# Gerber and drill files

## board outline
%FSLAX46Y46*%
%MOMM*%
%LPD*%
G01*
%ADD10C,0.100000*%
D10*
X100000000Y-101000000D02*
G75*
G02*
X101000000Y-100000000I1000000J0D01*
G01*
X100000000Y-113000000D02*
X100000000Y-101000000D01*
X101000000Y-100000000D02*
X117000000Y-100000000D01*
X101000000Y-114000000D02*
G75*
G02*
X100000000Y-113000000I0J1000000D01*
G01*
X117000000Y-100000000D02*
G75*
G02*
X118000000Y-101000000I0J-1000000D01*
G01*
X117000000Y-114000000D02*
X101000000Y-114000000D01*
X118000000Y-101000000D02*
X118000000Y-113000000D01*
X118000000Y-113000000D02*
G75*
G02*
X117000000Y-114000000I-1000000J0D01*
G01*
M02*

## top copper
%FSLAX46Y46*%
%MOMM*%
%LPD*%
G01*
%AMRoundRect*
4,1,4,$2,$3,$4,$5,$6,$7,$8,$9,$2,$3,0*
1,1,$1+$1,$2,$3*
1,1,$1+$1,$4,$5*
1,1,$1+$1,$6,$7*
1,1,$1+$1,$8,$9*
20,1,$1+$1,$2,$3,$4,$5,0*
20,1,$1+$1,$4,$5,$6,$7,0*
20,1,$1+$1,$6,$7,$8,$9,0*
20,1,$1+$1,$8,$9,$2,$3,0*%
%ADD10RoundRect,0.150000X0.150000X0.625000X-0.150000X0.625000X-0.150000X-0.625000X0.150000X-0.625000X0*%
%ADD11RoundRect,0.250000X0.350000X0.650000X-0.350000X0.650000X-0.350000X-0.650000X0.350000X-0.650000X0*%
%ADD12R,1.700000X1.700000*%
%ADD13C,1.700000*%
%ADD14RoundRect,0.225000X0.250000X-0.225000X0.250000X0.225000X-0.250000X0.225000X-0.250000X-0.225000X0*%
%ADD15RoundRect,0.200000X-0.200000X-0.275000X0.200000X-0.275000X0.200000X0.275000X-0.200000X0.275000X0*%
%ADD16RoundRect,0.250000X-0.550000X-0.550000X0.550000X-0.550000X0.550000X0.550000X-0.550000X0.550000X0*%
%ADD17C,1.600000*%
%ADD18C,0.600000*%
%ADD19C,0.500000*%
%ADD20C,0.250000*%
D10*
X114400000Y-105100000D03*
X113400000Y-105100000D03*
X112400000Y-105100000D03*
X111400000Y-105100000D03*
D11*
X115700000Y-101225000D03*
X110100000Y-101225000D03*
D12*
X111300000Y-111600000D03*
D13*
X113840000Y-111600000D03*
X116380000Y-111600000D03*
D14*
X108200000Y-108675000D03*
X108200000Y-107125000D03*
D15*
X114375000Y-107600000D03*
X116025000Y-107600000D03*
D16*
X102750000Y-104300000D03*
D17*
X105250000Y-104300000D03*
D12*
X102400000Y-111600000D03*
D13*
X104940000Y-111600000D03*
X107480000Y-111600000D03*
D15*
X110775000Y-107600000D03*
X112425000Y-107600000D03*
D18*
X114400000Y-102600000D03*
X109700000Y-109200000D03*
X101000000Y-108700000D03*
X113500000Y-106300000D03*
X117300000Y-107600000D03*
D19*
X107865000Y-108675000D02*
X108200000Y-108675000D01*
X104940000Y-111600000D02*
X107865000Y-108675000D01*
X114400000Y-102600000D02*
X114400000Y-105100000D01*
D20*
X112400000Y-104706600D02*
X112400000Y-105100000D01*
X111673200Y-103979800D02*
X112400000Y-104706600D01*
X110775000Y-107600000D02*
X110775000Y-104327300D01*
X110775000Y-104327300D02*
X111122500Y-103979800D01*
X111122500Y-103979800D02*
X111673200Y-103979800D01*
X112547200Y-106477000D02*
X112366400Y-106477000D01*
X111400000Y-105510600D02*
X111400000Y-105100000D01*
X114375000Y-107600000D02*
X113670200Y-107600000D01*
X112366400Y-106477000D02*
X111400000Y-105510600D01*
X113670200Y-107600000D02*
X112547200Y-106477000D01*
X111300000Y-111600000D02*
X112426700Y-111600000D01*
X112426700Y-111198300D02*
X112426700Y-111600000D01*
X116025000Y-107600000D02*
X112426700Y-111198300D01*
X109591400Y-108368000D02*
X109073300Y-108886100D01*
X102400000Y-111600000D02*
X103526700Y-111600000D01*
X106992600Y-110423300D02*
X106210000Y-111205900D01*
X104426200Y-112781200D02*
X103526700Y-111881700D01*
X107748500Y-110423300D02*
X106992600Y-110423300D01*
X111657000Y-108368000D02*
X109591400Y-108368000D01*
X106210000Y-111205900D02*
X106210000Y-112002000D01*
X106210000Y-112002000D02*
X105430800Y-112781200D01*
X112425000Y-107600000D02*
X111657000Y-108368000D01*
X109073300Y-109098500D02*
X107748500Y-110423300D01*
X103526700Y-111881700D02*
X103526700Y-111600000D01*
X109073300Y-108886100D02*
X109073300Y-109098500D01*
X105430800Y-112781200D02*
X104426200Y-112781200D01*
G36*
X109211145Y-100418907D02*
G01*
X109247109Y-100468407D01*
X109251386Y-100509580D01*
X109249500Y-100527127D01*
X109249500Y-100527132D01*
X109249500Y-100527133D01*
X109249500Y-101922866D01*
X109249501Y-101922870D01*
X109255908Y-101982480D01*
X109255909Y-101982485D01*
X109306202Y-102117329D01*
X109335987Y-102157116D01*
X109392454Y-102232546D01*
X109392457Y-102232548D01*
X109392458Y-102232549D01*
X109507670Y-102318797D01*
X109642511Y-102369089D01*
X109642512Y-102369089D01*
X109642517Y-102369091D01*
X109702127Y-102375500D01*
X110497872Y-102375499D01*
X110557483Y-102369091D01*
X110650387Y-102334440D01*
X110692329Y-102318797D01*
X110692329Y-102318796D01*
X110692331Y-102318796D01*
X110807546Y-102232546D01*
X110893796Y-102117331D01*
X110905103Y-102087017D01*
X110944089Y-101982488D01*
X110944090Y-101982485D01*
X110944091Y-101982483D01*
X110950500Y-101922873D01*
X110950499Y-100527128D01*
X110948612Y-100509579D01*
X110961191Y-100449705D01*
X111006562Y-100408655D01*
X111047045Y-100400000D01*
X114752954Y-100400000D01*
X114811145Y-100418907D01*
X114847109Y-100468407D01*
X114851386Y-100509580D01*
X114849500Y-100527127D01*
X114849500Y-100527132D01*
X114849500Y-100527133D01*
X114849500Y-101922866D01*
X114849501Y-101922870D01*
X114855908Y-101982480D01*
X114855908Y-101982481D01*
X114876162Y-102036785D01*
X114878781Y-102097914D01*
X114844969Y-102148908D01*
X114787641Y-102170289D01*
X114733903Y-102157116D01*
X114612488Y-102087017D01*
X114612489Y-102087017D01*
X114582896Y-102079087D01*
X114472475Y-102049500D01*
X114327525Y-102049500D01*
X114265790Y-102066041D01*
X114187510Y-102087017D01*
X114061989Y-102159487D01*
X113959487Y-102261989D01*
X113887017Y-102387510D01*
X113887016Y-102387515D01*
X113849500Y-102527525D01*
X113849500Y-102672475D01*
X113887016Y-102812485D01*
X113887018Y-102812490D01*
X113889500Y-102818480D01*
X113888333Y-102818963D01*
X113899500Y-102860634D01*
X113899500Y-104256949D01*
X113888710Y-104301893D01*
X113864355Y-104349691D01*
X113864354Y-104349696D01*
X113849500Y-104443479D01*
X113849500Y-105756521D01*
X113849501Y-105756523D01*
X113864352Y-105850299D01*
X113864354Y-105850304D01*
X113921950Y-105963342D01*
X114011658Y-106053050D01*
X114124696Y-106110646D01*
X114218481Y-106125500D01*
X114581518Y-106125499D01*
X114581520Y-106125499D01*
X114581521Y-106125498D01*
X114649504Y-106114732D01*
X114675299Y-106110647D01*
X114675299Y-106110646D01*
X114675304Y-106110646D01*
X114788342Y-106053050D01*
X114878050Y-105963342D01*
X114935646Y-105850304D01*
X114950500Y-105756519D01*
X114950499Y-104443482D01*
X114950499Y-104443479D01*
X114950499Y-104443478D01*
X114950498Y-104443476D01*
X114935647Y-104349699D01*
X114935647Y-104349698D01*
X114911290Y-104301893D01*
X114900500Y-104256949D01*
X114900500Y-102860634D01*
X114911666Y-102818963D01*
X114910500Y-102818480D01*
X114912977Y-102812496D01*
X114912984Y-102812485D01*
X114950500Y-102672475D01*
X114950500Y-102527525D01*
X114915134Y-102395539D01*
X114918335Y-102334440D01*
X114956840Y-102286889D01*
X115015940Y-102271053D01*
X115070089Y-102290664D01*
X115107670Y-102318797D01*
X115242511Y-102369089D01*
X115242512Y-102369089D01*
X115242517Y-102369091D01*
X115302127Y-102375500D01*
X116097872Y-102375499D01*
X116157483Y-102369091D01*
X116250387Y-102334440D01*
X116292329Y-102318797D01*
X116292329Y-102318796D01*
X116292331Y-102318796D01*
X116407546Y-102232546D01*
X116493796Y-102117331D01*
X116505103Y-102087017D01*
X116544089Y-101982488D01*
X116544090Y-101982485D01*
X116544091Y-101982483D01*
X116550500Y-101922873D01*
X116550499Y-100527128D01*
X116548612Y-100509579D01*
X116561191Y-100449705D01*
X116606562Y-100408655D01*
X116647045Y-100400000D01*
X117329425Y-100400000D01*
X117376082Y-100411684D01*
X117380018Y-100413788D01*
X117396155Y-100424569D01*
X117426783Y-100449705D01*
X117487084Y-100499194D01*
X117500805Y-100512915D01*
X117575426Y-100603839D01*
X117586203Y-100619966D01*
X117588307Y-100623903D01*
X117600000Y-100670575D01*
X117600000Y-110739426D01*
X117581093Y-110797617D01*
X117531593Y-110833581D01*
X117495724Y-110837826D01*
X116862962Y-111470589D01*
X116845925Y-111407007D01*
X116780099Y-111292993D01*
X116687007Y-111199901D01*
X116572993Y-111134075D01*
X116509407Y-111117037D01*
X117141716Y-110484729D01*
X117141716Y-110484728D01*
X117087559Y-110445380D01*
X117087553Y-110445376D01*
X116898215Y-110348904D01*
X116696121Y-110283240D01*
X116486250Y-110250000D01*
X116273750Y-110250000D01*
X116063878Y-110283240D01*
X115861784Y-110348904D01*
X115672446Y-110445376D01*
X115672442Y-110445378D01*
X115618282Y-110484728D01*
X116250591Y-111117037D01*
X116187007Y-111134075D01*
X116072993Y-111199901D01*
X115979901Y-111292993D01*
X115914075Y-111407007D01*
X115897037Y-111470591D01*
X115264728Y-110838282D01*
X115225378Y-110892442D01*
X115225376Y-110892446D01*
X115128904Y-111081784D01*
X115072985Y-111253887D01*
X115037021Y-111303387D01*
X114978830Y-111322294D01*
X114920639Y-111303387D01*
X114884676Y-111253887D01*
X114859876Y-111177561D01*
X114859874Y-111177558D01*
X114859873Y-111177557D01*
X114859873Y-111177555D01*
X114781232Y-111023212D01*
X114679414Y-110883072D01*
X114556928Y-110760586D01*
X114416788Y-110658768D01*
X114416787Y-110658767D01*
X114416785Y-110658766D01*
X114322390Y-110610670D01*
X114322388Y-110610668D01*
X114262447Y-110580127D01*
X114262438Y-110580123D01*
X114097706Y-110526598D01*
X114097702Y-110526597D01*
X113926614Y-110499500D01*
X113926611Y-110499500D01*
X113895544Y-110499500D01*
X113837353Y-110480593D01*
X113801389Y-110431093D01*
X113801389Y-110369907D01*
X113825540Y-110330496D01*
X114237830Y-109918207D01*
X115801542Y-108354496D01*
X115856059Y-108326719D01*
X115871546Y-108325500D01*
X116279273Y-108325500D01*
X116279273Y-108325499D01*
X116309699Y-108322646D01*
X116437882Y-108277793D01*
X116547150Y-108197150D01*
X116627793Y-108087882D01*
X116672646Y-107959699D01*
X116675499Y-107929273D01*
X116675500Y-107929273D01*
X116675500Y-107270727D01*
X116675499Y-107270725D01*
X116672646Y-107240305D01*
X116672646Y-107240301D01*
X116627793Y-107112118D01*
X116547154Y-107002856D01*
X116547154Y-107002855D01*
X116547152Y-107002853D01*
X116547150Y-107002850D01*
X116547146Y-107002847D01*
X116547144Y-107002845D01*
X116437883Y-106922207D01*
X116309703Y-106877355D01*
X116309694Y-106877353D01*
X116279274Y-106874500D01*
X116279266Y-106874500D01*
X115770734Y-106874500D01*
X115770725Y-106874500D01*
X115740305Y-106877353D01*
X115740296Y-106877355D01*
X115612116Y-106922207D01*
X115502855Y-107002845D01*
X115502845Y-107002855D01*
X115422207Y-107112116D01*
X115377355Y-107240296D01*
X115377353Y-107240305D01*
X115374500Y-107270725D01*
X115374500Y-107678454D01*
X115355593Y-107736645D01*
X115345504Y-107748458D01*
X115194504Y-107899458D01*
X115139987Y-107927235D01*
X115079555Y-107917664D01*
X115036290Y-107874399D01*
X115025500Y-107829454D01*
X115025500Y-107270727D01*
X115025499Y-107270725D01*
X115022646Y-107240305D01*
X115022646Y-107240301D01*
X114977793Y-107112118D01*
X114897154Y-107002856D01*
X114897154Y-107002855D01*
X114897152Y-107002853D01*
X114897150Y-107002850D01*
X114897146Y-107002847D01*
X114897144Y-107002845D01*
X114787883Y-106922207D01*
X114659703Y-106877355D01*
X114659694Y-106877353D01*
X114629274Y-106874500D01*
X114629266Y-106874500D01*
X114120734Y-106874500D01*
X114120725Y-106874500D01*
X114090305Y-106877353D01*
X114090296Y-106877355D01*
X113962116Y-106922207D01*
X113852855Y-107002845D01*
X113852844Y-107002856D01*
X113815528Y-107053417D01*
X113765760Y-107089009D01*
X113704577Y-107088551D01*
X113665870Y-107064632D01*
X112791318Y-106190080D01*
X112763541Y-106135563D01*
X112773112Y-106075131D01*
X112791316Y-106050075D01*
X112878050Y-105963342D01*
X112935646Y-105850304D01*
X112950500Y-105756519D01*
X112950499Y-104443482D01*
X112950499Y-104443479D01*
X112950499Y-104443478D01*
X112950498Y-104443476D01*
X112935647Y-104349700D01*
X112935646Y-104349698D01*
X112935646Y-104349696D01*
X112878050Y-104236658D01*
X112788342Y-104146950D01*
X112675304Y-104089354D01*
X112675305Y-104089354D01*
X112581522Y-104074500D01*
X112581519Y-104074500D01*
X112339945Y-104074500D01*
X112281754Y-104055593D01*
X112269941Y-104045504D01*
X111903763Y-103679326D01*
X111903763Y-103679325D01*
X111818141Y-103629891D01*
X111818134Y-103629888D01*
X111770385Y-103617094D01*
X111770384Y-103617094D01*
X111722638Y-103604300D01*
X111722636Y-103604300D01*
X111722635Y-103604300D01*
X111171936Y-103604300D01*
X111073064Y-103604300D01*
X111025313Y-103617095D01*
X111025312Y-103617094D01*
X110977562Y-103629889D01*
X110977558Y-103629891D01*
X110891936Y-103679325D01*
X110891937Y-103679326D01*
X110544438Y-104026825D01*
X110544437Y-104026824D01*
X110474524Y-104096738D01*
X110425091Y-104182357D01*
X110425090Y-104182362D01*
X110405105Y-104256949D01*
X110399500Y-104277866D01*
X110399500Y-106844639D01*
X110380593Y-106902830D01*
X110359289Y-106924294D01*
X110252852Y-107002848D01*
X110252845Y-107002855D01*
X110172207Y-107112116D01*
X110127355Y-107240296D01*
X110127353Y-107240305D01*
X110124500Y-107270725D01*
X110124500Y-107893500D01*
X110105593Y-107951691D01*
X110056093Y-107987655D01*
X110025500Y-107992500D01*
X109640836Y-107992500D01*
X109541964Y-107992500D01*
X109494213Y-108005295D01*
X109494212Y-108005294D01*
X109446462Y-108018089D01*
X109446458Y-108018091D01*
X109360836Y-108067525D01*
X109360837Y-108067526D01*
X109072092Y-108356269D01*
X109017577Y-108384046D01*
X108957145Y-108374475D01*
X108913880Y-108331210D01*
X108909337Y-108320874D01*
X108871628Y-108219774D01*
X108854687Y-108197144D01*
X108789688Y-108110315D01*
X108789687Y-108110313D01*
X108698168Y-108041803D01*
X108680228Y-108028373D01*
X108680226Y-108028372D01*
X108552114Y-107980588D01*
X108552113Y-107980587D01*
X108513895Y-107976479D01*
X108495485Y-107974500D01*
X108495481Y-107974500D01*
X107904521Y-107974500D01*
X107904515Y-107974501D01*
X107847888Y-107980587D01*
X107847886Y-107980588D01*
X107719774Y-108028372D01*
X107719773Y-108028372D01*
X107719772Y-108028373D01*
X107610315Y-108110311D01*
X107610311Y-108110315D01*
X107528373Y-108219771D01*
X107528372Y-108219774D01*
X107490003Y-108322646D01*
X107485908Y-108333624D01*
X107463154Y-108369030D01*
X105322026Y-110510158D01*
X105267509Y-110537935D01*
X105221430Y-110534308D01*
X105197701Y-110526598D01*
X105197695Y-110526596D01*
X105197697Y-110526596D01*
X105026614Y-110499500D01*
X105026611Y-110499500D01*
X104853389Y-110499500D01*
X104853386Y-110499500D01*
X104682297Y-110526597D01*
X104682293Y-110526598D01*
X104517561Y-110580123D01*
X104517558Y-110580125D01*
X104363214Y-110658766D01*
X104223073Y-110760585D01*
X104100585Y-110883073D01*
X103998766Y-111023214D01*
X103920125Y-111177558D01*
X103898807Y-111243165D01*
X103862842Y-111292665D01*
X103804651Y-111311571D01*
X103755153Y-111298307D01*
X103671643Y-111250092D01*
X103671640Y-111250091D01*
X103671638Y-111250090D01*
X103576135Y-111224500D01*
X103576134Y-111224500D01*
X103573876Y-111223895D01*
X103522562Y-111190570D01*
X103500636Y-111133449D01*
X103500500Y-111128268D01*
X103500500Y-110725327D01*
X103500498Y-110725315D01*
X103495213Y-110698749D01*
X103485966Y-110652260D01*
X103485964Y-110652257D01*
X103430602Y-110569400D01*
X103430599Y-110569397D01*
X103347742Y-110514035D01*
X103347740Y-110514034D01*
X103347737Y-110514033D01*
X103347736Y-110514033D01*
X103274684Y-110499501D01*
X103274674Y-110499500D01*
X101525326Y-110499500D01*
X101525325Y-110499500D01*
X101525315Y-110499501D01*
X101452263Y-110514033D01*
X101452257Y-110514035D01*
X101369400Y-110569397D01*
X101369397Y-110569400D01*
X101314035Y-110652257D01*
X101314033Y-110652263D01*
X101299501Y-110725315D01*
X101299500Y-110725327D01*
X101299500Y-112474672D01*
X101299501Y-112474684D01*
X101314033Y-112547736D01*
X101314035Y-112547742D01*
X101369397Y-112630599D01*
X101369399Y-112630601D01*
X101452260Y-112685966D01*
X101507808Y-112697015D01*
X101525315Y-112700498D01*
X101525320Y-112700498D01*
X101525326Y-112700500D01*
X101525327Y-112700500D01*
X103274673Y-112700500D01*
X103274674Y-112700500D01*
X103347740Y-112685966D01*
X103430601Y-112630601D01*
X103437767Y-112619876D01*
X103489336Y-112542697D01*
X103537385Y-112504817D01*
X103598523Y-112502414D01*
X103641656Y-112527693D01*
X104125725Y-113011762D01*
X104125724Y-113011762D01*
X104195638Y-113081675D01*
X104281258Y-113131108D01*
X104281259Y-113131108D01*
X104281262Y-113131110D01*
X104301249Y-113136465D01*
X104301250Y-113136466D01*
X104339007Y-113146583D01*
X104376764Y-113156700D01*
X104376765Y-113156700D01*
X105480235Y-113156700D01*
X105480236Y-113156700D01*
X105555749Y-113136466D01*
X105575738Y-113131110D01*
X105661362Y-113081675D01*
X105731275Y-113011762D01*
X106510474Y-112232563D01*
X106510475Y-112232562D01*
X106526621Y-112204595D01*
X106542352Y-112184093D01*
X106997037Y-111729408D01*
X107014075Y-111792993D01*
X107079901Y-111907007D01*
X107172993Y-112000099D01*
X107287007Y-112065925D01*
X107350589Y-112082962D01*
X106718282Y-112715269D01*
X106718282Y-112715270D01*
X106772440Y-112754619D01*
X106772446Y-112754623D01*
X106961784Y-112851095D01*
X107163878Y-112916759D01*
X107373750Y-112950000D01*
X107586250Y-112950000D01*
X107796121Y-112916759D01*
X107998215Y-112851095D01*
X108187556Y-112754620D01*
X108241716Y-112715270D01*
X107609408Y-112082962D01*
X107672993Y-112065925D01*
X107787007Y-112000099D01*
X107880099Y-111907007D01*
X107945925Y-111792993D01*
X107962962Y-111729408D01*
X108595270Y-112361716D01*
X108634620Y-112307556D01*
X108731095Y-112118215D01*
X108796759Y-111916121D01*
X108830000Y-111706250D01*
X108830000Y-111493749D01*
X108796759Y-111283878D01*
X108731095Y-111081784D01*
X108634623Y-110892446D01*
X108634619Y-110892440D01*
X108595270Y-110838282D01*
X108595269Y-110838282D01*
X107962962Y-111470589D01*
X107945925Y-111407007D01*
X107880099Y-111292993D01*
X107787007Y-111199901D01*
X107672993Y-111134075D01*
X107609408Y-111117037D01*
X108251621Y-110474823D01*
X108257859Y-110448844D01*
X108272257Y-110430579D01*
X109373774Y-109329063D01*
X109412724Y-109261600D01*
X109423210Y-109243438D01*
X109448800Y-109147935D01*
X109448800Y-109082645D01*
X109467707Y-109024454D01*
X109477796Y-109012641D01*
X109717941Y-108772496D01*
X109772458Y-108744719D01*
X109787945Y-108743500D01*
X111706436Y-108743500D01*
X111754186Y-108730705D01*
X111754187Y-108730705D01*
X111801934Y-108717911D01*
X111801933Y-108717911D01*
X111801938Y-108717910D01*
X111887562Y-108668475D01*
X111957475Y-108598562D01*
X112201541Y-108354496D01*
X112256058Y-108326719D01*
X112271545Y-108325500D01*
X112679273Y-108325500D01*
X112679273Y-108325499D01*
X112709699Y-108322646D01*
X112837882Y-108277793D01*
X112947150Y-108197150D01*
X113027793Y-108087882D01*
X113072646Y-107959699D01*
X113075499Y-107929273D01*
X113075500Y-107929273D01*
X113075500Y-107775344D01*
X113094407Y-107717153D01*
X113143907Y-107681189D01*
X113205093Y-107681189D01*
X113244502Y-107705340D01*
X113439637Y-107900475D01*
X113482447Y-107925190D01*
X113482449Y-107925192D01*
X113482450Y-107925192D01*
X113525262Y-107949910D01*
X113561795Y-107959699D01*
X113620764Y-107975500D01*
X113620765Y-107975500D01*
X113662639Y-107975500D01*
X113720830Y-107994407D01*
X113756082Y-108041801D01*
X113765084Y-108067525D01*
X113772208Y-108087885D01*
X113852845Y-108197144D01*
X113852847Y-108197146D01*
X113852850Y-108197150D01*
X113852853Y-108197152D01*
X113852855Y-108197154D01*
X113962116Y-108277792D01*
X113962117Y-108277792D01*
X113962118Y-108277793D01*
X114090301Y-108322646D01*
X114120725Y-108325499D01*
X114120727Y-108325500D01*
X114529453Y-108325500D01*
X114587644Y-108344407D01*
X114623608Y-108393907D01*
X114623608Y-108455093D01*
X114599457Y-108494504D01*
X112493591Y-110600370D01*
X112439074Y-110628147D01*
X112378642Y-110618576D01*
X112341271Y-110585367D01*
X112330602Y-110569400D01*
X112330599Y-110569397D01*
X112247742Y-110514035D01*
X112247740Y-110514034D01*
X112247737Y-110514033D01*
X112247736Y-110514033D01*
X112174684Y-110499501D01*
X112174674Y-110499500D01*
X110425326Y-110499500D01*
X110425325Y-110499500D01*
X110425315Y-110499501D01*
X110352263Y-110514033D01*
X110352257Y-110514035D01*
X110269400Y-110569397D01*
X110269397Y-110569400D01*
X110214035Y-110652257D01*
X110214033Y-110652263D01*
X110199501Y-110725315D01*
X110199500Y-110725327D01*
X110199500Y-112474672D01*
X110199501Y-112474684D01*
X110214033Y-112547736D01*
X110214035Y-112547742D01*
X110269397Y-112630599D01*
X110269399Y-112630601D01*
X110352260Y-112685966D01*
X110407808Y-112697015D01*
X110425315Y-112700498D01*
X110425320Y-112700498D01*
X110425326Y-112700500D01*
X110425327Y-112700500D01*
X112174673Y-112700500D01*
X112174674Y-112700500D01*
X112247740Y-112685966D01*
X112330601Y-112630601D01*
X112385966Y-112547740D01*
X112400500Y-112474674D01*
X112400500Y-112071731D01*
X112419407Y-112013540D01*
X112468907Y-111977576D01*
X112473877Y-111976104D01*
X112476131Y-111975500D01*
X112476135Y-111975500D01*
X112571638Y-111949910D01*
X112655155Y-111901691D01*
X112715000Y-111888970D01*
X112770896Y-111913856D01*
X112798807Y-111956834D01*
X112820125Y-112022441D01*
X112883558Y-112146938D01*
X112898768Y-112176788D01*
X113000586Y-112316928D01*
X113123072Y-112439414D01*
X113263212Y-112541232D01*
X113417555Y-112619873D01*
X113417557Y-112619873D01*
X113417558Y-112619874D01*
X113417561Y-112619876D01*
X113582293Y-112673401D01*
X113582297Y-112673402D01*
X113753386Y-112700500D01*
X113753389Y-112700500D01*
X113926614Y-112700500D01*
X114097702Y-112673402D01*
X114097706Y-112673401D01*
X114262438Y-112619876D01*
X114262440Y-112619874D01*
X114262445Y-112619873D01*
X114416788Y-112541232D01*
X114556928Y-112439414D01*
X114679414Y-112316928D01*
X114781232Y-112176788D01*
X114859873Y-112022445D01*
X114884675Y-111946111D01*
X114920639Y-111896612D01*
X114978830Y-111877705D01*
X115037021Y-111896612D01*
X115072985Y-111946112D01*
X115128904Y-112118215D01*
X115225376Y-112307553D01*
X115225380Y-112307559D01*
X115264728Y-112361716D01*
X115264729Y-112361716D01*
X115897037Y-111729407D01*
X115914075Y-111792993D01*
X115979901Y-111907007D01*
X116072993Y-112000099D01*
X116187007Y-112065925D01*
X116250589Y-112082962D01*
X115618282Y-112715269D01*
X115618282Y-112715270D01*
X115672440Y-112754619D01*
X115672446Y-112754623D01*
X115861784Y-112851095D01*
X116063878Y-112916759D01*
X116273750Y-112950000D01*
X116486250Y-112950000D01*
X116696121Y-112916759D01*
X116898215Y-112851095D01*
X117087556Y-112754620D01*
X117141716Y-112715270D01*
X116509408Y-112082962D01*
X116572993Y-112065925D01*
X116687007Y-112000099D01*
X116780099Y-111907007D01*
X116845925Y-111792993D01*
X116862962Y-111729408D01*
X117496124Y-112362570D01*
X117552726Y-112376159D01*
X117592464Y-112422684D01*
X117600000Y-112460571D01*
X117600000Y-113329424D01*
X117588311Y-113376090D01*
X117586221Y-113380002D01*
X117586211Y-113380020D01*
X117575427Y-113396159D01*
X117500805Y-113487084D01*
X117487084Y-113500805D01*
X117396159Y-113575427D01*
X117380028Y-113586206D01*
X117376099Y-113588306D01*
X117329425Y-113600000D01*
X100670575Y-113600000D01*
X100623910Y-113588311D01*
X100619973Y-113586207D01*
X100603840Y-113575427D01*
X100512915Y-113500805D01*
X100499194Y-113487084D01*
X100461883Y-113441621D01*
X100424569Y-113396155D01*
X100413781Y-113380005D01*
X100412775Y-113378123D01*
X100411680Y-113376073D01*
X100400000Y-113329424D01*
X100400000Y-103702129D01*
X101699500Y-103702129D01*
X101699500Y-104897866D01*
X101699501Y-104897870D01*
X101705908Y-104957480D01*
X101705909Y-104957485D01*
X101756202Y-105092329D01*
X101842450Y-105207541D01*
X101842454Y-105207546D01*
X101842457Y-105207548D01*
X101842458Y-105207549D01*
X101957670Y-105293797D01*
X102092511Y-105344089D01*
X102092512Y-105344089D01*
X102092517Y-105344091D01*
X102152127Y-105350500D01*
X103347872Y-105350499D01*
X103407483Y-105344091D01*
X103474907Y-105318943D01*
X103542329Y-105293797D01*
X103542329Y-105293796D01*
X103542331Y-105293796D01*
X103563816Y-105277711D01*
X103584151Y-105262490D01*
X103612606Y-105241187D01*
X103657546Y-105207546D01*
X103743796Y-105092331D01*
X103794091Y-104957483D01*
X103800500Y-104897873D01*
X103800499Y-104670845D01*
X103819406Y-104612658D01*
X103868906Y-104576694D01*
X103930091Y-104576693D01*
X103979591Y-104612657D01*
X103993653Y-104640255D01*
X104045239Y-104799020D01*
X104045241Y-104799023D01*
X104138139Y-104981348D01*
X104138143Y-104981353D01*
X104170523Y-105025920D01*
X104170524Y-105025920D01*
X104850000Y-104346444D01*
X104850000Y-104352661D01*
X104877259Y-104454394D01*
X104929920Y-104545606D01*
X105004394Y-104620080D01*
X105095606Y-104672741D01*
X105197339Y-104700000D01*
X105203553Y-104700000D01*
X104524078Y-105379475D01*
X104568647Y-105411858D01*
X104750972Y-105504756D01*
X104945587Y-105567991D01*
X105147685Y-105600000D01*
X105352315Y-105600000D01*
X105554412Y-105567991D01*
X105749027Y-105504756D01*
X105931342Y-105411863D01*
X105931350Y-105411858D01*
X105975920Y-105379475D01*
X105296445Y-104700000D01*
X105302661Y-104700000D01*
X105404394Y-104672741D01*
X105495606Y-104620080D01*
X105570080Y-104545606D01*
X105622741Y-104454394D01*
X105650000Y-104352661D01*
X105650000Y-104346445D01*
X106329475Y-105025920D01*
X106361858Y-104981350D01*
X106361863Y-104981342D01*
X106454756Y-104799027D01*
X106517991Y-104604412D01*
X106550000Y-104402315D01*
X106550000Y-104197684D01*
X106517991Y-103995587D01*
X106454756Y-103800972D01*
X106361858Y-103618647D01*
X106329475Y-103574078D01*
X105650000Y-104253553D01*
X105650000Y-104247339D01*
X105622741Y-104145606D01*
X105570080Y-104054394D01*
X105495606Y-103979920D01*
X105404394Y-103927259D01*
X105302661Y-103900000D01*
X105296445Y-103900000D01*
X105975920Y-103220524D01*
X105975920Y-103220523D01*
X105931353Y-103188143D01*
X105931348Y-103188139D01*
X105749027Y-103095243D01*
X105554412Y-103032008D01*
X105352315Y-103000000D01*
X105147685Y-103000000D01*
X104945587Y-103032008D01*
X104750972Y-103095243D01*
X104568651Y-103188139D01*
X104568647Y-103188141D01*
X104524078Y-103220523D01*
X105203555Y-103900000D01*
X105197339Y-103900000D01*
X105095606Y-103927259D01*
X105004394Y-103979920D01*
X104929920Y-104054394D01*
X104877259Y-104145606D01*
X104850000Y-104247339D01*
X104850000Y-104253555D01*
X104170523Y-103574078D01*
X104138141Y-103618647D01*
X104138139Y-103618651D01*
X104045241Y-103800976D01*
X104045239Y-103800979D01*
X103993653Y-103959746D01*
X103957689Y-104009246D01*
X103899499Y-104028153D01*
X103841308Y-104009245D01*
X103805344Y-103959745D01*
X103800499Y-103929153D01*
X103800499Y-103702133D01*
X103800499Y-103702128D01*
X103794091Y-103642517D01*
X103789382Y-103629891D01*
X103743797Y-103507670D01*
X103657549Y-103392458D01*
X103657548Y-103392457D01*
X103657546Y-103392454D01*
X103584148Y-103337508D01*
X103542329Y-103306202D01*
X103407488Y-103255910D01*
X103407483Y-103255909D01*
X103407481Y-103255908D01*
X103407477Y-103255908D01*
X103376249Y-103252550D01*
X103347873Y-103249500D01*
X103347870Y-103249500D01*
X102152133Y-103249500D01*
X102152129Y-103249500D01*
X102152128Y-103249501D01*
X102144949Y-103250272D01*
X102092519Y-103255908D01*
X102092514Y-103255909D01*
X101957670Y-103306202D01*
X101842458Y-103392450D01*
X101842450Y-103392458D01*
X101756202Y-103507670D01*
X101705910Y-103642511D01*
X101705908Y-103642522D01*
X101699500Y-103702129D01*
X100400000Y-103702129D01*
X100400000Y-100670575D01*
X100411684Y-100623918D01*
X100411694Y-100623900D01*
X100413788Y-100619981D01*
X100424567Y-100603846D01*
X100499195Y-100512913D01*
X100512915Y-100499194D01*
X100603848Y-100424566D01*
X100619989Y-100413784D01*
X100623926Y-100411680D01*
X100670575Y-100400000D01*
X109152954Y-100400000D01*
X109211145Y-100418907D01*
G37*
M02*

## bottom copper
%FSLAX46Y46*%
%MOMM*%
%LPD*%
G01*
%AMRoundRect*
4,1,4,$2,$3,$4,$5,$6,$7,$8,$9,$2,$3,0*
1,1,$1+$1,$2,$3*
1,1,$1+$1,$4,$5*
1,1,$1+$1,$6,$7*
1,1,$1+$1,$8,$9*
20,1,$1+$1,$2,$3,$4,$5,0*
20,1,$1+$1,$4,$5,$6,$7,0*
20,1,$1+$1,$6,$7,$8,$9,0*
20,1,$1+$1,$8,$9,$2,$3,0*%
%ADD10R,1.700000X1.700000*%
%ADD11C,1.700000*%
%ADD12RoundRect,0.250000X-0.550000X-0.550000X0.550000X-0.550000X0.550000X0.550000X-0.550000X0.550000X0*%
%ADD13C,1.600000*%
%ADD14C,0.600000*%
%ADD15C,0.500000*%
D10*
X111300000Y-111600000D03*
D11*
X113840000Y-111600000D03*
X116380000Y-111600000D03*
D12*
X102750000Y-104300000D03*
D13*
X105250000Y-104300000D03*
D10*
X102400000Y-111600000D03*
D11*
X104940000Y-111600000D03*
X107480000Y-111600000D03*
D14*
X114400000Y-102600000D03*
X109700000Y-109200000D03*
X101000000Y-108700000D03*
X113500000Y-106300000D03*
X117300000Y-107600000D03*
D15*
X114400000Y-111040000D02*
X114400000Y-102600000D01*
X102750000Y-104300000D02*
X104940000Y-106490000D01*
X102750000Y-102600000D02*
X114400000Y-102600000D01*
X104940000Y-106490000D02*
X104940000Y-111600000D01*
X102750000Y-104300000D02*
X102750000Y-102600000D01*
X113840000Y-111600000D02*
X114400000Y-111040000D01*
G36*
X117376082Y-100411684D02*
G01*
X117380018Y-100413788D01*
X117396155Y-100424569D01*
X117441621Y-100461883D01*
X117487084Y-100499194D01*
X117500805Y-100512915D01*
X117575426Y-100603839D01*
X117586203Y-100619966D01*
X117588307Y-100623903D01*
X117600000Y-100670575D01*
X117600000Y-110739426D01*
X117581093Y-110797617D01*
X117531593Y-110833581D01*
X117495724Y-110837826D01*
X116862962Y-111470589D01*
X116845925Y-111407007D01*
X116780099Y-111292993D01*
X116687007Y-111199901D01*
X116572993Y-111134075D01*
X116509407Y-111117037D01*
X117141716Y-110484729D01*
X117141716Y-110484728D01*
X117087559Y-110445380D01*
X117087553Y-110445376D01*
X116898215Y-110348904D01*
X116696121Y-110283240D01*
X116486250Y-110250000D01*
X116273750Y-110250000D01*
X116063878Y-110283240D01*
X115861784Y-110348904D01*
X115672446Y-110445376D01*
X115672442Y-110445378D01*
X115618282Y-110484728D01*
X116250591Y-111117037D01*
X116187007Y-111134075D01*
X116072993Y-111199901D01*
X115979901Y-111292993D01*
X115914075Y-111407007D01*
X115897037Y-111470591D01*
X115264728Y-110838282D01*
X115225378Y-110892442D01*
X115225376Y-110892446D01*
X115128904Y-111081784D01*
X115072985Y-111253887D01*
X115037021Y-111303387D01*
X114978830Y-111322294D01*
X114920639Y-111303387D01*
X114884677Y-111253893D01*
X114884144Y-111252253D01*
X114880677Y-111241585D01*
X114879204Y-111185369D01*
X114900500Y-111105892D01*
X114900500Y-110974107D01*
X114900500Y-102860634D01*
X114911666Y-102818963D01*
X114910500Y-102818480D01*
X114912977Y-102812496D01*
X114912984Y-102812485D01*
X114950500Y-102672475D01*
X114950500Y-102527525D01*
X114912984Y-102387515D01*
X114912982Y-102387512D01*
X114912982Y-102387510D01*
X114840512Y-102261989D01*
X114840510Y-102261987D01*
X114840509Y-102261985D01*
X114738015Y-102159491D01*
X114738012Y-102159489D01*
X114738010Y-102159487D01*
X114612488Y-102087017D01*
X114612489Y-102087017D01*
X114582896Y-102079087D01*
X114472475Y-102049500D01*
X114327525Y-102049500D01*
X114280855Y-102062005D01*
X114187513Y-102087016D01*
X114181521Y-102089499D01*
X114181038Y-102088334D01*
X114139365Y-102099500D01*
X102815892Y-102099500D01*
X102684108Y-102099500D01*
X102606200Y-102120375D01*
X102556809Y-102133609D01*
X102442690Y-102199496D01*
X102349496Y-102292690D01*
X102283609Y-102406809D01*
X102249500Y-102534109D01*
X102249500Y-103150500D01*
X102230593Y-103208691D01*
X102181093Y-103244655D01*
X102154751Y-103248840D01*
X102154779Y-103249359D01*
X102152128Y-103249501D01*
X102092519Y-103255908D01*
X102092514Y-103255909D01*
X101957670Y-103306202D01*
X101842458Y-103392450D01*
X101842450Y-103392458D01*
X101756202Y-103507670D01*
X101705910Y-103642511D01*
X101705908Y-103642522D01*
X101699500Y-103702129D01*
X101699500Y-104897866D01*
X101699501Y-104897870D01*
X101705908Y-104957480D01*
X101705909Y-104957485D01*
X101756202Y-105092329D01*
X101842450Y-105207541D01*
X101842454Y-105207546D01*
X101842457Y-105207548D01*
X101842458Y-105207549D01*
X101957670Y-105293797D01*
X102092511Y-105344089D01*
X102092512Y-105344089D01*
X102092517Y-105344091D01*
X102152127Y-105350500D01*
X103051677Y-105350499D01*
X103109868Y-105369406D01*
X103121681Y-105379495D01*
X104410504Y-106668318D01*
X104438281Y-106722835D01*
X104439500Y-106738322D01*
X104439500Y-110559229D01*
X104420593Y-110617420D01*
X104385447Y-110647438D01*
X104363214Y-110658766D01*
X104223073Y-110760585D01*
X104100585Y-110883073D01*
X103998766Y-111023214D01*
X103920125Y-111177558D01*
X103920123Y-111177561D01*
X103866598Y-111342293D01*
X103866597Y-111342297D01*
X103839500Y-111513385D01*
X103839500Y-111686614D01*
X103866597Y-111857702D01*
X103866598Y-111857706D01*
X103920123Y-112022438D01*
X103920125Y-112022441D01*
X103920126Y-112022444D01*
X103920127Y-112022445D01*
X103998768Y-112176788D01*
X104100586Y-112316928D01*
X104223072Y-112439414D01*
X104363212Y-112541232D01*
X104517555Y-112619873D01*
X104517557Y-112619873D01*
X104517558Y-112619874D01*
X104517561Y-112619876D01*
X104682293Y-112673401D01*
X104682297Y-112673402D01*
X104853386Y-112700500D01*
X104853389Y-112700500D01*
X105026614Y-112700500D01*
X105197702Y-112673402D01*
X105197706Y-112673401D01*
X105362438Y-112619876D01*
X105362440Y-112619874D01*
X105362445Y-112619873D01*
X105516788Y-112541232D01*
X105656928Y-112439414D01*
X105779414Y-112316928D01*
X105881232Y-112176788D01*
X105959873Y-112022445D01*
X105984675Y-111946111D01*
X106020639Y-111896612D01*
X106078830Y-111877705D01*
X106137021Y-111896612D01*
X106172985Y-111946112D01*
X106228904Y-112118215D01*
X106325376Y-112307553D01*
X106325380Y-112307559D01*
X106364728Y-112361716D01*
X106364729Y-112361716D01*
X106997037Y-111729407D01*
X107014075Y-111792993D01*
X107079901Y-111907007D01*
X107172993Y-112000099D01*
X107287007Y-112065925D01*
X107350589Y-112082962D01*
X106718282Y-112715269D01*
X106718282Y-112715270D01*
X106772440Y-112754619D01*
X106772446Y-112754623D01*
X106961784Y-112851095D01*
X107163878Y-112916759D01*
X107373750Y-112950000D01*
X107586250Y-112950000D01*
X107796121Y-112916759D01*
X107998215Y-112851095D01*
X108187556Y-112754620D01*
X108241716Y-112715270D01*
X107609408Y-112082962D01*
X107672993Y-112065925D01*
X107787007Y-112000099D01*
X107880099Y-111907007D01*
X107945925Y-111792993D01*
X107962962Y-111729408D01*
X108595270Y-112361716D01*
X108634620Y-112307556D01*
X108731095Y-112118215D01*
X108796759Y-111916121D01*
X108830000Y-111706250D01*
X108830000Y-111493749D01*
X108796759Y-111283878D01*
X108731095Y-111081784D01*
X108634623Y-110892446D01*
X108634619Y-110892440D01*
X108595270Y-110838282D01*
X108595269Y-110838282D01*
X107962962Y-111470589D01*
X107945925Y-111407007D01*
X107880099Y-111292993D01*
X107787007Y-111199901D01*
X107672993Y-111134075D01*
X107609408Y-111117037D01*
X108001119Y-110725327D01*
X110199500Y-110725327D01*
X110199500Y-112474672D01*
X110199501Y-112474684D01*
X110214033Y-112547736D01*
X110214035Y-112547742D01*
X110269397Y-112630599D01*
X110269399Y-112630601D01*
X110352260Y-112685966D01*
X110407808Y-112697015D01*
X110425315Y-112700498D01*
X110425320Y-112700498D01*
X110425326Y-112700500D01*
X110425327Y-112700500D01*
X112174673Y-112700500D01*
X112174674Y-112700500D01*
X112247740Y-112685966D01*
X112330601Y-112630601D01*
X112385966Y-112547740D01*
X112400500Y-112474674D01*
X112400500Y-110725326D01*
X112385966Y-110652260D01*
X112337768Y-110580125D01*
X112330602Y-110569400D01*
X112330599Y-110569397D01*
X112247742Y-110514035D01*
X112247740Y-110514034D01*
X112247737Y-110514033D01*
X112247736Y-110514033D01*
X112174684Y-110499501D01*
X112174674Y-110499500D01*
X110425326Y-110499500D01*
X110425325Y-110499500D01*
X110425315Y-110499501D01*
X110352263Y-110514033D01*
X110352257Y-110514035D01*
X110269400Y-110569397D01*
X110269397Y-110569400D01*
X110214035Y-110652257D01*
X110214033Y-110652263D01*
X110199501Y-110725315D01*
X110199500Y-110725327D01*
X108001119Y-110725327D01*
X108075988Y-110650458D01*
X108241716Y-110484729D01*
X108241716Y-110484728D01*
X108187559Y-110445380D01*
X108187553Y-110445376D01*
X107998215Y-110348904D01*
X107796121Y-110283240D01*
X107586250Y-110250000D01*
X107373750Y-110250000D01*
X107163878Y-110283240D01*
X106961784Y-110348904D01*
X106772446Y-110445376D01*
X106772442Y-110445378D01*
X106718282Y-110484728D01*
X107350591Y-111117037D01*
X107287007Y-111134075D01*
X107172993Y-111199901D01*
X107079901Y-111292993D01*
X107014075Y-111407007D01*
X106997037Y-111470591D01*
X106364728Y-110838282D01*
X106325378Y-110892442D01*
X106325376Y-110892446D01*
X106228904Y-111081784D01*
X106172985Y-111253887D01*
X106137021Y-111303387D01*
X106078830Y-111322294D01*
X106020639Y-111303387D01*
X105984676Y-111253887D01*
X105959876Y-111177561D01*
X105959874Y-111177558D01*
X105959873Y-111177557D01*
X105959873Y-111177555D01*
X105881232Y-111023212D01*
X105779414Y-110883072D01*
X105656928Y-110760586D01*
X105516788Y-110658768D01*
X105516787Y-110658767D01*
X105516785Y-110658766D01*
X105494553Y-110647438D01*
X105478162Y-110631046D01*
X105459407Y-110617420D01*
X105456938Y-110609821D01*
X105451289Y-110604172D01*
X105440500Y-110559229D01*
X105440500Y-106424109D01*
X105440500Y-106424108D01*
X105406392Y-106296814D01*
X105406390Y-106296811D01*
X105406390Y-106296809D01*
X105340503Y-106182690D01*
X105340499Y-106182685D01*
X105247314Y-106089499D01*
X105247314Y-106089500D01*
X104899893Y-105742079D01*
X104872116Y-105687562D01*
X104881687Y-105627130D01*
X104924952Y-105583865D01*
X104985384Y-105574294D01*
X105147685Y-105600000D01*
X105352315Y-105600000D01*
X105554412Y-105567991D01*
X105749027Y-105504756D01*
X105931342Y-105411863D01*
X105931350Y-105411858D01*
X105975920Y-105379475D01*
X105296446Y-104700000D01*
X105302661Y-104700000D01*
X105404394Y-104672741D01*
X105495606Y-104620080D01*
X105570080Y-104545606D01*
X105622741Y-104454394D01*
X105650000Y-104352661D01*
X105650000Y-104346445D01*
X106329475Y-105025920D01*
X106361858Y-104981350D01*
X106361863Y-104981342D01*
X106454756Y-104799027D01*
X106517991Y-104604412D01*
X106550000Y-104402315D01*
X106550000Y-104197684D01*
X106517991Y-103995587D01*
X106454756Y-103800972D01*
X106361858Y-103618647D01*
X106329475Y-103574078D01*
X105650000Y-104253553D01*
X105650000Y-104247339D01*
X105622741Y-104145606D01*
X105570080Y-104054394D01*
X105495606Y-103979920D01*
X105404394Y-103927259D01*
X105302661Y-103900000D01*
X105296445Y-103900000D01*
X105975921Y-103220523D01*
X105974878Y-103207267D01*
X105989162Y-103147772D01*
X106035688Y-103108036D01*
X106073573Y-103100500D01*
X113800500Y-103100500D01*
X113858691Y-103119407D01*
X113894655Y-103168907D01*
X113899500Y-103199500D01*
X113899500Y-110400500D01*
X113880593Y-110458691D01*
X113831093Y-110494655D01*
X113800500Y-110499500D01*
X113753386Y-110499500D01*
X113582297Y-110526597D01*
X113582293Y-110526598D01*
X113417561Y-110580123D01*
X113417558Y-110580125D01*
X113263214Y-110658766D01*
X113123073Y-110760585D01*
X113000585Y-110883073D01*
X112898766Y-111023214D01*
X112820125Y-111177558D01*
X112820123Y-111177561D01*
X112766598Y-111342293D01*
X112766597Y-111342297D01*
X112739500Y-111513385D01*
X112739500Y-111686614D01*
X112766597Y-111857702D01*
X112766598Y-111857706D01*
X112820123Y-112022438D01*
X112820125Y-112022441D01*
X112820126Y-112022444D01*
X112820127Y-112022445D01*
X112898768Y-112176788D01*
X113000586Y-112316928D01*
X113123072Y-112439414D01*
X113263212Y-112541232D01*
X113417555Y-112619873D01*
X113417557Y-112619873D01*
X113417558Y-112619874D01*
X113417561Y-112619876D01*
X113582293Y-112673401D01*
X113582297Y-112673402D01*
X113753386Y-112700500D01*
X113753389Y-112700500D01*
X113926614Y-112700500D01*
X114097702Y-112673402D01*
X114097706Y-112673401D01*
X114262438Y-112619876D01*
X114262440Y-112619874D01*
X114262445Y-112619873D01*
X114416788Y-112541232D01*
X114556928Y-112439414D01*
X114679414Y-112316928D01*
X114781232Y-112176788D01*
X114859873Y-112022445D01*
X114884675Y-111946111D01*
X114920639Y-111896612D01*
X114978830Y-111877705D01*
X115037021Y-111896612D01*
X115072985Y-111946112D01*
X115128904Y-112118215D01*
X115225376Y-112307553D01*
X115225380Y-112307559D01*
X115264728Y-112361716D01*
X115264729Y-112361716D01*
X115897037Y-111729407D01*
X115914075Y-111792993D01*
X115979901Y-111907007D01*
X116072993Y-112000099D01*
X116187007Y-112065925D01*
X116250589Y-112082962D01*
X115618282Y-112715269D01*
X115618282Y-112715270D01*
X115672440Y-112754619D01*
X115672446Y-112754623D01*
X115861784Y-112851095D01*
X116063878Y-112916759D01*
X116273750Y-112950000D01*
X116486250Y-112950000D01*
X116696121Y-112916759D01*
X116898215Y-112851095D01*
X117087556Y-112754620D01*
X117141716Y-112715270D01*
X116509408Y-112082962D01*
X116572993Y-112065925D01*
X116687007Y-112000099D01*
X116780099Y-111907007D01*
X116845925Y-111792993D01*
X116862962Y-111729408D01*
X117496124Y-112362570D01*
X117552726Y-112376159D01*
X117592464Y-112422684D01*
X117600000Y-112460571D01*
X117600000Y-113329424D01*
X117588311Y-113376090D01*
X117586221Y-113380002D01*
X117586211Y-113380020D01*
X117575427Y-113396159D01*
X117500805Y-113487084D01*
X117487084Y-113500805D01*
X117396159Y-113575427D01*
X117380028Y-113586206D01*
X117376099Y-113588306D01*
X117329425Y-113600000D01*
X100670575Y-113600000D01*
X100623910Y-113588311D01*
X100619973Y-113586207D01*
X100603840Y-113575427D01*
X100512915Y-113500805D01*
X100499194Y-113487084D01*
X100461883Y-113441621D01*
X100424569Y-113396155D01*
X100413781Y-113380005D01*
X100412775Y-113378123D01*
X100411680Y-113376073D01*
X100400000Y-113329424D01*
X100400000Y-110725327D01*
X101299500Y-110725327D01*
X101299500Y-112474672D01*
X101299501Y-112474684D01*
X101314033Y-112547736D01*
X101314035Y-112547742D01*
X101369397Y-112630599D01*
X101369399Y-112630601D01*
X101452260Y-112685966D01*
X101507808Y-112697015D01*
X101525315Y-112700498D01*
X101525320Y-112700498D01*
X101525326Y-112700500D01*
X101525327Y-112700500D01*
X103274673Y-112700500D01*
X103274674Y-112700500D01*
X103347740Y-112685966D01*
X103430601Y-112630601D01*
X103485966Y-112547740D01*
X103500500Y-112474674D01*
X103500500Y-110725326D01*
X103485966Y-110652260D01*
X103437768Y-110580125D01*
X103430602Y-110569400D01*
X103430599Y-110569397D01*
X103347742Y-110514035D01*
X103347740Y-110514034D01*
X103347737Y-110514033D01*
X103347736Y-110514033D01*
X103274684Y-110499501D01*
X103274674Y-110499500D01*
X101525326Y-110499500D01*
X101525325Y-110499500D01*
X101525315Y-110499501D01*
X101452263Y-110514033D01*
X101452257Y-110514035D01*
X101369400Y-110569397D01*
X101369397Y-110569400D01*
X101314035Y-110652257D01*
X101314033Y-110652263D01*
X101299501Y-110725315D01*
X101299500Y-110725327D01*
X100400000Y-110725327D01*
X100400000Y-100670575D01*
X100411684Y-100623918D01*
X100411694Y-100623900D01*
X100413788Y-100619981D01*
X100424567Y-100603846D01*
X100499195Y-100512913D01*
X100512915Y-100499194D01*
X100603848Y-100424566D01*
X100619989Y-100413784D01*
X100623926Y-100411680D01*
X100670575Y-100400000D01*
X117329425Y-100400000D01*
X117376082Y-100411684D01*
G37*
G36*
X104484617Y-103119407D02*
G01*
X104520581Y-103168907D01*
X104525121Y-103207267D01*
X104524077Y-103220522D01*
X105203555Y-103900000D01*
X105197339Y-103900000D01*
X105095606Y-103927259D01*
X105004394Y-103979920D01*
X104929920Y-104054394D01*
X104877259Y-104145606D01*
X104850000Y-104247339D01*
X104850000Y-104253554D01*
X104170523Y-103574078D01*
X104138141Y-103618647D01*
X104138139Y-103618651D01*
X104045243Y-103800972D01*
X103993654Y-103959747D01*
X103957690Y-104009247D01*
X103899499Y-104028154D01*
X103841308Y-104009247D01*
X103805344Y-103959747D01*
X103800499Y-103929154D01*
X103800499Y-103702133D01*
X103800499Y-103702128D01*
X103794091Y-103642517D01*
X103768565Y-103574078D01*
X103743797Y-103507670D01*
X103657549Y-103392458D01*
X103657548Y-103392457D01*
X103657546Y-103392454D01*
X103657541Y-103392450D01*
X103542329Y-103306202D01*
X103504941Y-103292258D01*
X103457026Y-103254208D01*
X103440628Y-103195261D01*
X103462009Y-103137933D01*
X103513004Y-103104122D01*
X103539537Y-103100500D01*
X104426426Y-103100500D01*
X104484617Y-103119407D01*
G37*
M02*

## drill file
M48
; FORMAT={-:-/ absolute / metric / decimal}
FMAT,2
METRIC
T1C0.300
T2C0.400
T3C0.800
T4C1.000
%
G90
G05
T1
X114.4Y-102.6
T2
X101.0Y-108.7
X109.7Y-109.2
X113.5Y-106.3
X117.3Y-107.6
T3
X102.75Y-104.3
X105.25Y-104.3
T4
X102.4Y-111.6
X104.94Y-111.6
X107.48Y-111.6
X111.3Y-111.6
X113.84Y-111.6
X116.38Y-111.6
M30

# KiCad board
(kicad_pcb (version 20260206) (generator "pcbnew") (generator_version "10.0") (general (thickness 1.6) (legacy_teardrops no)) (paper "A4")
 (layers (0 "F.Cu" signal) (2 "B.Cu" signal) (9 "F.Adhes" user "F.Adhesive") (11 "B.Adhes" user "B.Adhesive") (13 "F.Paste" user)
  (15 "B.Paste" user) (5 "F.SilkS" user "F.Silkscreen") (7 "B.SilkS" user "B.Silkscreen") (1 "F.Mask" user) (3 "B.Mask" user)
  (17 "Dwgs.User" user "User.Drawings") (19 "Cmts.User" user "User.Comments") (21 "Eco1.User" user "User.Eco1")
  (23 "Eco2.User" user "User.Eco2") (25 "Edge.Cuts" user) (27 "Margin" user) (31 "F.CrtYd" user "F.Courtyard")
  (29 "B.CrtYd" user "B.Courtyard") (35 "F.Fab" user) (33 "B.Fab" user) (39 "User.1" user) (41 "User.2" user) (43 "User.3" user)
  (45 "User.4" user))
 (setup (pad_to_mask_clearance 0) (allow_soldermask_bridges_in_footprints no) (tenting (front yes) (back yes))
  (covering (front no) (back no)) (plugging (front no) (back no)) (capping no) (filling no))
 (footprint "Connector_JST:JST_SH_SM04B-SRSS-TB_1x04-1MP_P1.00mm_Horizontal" (layer "F.Cu") (at 112.9 103.1 180)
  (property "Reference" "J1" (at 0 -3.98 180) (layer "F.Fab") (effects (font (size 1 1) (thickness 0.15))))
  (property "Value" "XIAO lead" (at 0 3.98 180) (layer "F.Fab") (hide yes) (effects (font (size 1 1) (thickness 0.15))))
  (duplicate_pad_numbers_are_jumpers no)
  (pad "1" smd roundrect (at -1.5 -2 180) (size 0.6 1.55) (layers "F.Cu" "F.Mask" "F.Paste") (roundrect_rratio 0.25) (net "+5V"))
  (pad "2" smd roundrect (at -0.5 -2 180) (size 0.6 1.55) (layers "F.Cu" "F.Mask" "F.Paste") (roundrect_rratio 0.25) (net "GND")
   (zone_connect 2))
  (pad "3" smd roundrect (at 0.5 -2 180) (size 0.6 1.55) (layers "F.Cu" "F.Mask" "F.Paste") (roundrect_rratio 0.25) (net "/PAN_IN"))
  (pad "4" smd roundrect (at 1.5 -2 180) (size 0.6 1.55) (layers "F.Cu" "F.Mask" "F.Paste") (roundrect_rratio 0.25) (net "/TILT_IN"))
  (pad "MP" smd roundrect (at -2.8 1.875 180) (size 1.2 1.8) (layers "F.Cu" "F.Mask" "F.Paste") (roundrect_rratio 0.208333))
  (pad "MP" smd roundrect (at 2.8 1.875 180) (size 1.2 1.8) (layers "F.Cu" "F.Mask" "F.Paste") (roundrect_rratio 0.208333)))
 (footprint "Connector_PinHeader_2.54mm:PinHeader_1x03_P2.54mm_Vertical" (layer "F.Cu") (at 111.3 111.6 90)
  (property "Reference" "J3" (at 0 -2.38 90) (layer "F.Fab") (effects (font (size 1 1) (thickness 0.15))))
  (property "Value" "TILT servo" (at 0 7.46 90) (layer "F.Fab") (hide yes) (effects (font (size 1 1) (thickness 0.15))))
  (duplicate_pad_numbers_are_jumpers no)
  (pad "1" thru_hole rect (at 0 0 90) (size 1.7 1.7) (drill 1) (layers "*.Cu" "*.Mask") (remove_unused_layers no) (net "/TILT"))
  (pad "2" thru_hole circle (at 0 2.54 90) (size 1.7 1.7) (drill 1) (layers "*.Cu" "*.Mask") (remove_unused_layers no) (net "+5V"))
  (pad "3" thru_hole circle (at 0 5.08 90) (size 1.7 1.7) (drill 1) (layers "*.Cu" "*.Mask") (remove_unused_layers no) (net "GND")))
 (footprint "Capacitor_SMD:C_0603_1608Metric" (layer "F.Cu") (at 108.2 107.9 90)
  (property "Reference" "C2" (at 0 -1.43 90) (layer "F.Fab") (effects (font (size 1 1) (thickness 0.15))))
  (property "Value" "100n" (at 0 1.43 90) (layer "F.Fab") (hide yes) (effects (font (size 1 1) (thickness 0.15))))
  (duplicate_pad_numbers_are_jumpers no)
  (pad "1" smd roundrect (at -0.775 0 90) (size 0.9 0.95) (layers "F.Cu" "F.Mask" "F.Paste") (roundrect_rratio 0.25) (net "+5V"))
  (pad "2" smd roundrect (at 0.775 0 90) (size 0.9 0.95) (layers "F.Cu" "F.Mask" "F.Paste") (roundrect_rratio 0.25) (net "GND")
   (zone_connect 2)))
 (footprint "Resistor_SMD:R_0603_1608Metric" (layer "F.Cu") (at 115.2 107.6)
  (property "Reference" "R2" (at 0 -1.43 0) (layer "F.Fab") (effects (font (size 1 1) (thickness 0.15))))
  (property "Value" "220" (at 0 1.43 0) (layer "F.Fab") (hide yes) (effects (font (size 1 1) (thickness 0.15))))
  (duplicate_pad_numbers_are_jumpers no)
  (pad "1" smd roundrect (at -0.825 0) (size 0.8 0.95) (layers "F.Cu" "F.Mask" "F.Paste") (roundrect_rratio 0.25) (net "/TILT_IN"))
  (pad "2" smd roundrect (at 0.825 0) (size 0.8 0.95) (layers "F.Cu" "F.Mask" "F.Paste") (roundrect_rratio 0.25) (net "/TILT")))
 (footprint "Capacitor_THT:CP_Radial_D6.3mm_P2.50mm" (layer "F.Cu") (at 102.75 104.3)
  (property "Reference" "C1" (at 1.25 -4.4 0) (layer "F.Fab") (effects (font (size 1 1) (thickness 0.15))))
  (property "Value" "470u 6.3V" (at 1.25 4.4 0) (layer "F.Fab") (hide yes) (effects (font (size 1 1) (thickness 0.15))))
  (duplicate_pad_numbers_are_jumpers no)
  (pad "1" thru_hole roundrect (at 0 0) (size 1.6 1.6) (drill 0.8) (layers "*.Cu" "*.Mask") (remove_unused_layers no)
   (roundrect_rratio 0.15625) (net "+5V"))
  (pad "2" thru_hole circle (at 2.5 0) (size 1.6 1.6) (drill 0.8) (layers "*.Cu" "*.Mask") (remove_unused_layers no) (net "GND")))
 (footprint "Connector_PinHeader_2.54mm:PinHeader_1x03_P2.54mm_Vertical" (layer "F.Cu") (at 102.4 111.6 90)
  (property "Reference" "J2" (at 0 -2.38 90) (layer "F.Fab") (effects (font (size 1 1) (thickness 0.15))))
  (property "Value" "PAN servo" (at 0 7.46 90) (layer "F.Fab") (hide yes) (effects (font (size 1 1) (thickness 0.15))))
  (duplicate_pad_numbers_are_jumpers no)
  (pad "1" thru_hole rect (at 0 0 90) (size 1.7 1.7) (drill 1) (layers "*.Cu" "*.Mask") (remove_unused_layers no) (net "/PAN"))
  (pad "2" thru_hole circle (at 0 2.54 90) (size 1.7 1.7) (drill 1) (layers "*.Cu" "*.Mask") (remove_unused_layers no) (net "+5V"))
  (pad "3" thru_hole circle (at 0 5.08 90) (size 1.7 1.7) (drill 1) (layers "*.Cu" "*.Mask") (remove_unused_layers no) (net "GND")))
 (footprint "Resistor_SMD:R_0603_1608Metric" (layer "F.Cu") (at 111.6 107.6)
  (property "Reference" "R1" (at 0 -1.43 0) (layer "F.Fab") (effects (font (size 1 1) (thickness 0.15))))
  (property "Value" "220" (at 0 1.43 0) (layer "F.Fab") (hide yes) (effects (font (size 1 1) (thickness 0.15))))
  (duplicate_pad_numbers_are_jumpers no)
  (pad "1" smd roundrect (at -0.825 0) (size 0.8 0.95) (layers "F.Cu" "F.Mask" "F.Paste") (roundrect_rratio 0.25) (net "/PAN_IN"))
  (pad "2" smd roundrect (at 0.825 0) (size 0.8 0.95) (layers "F.Cu" "F.Mask" "F.Paste") (roundrect_rratio 0.25) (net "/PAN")))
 (gr_arc (start 100 101) (mid 100.292893 100.292893) (end 101 100) (stroke (width 0.1) (type default)) (layer "Edge.Cuts"))
 (gr_line (start 100 113) (end 100 101) (stroke (width 0.1) (type default)) (layer "Edge.Cuts"))
 (gr_line (start 101 100) (end 117 100) (stroke (width 0.1) (type default)) (layer "Edge.Cuts"))
 (gr_arc (start 101 114) (mid 100.292893 113.707107) (end 100 113) (stroke (width 0.1) (type default)) (layer "Edge.Cuts"))
 (gr_arc (start 117 100) (mid 117.707107 100.292893) (end 118 101) (stroke (width 0.1) (type default)) (layer "Edge.Cuts"))
 (gr_line (start 117 114) (end 101 114) (stroke (width 0.1) (type default)) (layer "Edge.Cuts"))
 (gr_line (start 118 101) (end 118 113) (stroke (width 0.1) (type default)) (layer "Edge.Cuts"))
 (gr_arc (start 118 113) (mid 117.707107 113.707107) (end 117 114) (stroke (width 0.1) (type default)) (layer "Edge.Cuts"))
 (segment (start 107.865 108.675) (end 108.2 108.675) (width 0.5) (layer "F.Cu") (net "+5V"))
 (segment (start 104.94 111.6) (end 107.865 108.675) (width 0.5) (layer "F.Cu") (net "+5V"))
 (segment (start 114.4 102.6) (end 114.4 105.1) (width 0.5) (locked yes) (layer "F.Cu") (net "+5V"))
 (via (at 114.4 102.6) (size 0.6) (drill 0.3) (layers "F.Cu" "B.Cu") (locked yes) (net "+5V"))
 (segment (start 114.4 111.04) (end 114.4 102.6) (width 0.5) (layer "B.Cu") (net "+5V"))
 (segment (start 102.75 104.3) (end 104.94 106.49) (width 0.5) (layer "B.Cu") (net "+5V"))
 (segment (start 102.75 102.6) (end 114.4 102.6) (width 0.5) (locked yes) (layer "B.Cu") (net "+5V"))
 (segment (start 104.94 106.49) (end 104.94 111.6) (width 0.5) (layer "B.Cu") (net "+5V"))
 (segment (start 102.75 104.3) (end 102.75 102.6) (width 0.5) (locked yes) (layer "B.Cu") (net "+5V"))
 (segment (start 113.84 111.6) (end 114.4 111.04) (width 0.5) (layer "B.Cu") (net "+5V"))
 (via (at 109.7 109.2) (size 0.6) (drill 0.4) (layers "F.Cu" "B.Cu") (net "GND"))
 (via (at 101 108.7) (size 0.6) (drill 0.4) (layers "F.Cu" "B.Cu") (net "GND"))
 (via (at 113.5 106.3) (size 0.6) (drill 0.4) (layers "F.Cu" "B.Cu") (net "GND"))
 (via (at 117.3 107.6) (size 0.6) (drill 0.4) (layers "F.Cu" "B.Cu") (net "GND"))
 (segment (start 112.4 104.7066) (end 112.4 105.1) (width 0.25) (layer "F.Cu") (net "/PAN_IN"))
 (segment (start 111.6732 103.9798) (end 112.4 104.7066) (width 0.25) (layer "F.Cu") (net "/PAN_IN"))
 (segment (start 110.775 107.6) (end 110.775 104.3273) (width 0.25) (layer "F.Cu") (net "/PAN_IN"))
 (segment (start 110.775 104.3273) (end 111.1225 103.9798) (width 0.25) (layer "F.Cu") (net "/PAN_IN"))
 (segment (start 111.1225 103.9798) (end 111.6732 103.9798) (width 0.25) (layer "F.Cu") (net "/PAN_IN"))
 (segment (start 112.5472 106.477) (end 112.3664 106.477) (width 0.25) (layer "F.Cu") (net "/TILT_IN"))
 (segment (start 111.4 105.5106) (end 111.4 105.1) (width 0.25) (layer "F.Cu") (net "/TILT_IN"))
 (segment (start 114.375 107.6) (end 113.6702 107.6) (width 0.25) (layer "F.Cu") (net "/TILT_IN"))
 (segment (start 112.3664 106.477) (end 111.4 105.5106) (width 0.25) (layer "F.Cu") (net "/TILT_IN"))
 (segment (start 113.6702 107.6) (end 112.5472 106.477) (width 0.25) (layer "F.Cu") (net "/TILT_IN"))
 (segment (start 111.3 111.6) (end 112.4267 111.6) (width 0.25) (layer "F.Cu") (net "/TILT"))
 (segment (start 112.4267 111.1983) (end 112.4267 111.6) (width 0.25) (layer "F.Cu") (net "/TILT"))
 (segment (start 116.025 107.6) (end 112.4267 111.1983) (width 0.25) (layer "F.Cu") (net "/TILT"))
 (segment (start 109.5914 108.368) (end 109.0733 108.8861) (width 0.25) (layer "F.Cu") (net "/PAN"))
 (segment (start 102.4 111.6) (end 103.5267 111.6) (width 0.25) (layer "F.Cu") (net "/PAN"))
 (segment (start 106.9926 110.4233) (end 106.21 111.2059) (width 0.25) (layer "F.Cu") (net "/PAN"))
 (segment (start 104.4262 112.7812) (end 103.5267 111.8817) (width 0.25) (layer "F.Cu") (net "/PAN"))
 (segment (start 107.7485 110.4233) (end 106.9926 110.4233) (width 0.25) (layer "F.Cu") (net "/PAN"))
 (segment (start 111.657 108.368) (end 109.5914 108.368) (width 0.25) (layer "F.Cu") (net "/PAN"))
 (segment (start 106.21 111.2059) (end 106.21 112.002) (width 0.25) (layer "F.Cu") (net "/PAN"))
 (segment (start 106.21 112.002) (end 105.4308 112.7812) (width 0.25) (layer "F.Cu") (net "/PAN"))
 (segment (start 112.425 107.6) (end 111.657 108.368) (width 0.25) (layer "F.Cu") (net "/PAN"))
 (segment (start 109.0733 109.0985) (end 107.7485 110.4233) (width 0.25) (layer "F.Cu") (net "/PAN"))
 (segment (start 103.5267 111.8817) (end 103.5267 111.6) (width 0.25) (layer "F.Cu") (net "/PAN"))
 (segment (start 109.0733 108.8861) (end 109.0733 109.0985) (width 0.25) (layer "F.Cu") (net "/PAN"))
 (segment (start 105.4308 112.7812) (end 104.4262 112.7812) (width 0.25) (layer "F.Cu") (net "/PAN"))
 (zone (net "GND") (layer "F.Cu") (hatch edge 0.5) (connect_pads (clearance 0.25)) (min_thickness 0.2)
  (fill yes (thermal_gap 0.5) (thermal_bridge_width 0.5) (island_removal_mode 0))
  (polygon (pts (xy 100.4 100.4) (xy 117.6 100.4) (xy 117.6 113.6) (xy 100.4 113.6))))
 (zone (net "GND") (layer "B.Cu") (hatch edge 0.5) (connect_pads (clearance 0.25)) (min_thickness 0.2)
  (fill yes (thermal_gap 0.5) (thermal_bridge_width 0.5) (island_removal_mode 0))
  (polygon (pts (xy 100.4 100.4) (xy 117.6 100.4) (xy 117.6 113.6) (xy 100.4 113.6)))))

